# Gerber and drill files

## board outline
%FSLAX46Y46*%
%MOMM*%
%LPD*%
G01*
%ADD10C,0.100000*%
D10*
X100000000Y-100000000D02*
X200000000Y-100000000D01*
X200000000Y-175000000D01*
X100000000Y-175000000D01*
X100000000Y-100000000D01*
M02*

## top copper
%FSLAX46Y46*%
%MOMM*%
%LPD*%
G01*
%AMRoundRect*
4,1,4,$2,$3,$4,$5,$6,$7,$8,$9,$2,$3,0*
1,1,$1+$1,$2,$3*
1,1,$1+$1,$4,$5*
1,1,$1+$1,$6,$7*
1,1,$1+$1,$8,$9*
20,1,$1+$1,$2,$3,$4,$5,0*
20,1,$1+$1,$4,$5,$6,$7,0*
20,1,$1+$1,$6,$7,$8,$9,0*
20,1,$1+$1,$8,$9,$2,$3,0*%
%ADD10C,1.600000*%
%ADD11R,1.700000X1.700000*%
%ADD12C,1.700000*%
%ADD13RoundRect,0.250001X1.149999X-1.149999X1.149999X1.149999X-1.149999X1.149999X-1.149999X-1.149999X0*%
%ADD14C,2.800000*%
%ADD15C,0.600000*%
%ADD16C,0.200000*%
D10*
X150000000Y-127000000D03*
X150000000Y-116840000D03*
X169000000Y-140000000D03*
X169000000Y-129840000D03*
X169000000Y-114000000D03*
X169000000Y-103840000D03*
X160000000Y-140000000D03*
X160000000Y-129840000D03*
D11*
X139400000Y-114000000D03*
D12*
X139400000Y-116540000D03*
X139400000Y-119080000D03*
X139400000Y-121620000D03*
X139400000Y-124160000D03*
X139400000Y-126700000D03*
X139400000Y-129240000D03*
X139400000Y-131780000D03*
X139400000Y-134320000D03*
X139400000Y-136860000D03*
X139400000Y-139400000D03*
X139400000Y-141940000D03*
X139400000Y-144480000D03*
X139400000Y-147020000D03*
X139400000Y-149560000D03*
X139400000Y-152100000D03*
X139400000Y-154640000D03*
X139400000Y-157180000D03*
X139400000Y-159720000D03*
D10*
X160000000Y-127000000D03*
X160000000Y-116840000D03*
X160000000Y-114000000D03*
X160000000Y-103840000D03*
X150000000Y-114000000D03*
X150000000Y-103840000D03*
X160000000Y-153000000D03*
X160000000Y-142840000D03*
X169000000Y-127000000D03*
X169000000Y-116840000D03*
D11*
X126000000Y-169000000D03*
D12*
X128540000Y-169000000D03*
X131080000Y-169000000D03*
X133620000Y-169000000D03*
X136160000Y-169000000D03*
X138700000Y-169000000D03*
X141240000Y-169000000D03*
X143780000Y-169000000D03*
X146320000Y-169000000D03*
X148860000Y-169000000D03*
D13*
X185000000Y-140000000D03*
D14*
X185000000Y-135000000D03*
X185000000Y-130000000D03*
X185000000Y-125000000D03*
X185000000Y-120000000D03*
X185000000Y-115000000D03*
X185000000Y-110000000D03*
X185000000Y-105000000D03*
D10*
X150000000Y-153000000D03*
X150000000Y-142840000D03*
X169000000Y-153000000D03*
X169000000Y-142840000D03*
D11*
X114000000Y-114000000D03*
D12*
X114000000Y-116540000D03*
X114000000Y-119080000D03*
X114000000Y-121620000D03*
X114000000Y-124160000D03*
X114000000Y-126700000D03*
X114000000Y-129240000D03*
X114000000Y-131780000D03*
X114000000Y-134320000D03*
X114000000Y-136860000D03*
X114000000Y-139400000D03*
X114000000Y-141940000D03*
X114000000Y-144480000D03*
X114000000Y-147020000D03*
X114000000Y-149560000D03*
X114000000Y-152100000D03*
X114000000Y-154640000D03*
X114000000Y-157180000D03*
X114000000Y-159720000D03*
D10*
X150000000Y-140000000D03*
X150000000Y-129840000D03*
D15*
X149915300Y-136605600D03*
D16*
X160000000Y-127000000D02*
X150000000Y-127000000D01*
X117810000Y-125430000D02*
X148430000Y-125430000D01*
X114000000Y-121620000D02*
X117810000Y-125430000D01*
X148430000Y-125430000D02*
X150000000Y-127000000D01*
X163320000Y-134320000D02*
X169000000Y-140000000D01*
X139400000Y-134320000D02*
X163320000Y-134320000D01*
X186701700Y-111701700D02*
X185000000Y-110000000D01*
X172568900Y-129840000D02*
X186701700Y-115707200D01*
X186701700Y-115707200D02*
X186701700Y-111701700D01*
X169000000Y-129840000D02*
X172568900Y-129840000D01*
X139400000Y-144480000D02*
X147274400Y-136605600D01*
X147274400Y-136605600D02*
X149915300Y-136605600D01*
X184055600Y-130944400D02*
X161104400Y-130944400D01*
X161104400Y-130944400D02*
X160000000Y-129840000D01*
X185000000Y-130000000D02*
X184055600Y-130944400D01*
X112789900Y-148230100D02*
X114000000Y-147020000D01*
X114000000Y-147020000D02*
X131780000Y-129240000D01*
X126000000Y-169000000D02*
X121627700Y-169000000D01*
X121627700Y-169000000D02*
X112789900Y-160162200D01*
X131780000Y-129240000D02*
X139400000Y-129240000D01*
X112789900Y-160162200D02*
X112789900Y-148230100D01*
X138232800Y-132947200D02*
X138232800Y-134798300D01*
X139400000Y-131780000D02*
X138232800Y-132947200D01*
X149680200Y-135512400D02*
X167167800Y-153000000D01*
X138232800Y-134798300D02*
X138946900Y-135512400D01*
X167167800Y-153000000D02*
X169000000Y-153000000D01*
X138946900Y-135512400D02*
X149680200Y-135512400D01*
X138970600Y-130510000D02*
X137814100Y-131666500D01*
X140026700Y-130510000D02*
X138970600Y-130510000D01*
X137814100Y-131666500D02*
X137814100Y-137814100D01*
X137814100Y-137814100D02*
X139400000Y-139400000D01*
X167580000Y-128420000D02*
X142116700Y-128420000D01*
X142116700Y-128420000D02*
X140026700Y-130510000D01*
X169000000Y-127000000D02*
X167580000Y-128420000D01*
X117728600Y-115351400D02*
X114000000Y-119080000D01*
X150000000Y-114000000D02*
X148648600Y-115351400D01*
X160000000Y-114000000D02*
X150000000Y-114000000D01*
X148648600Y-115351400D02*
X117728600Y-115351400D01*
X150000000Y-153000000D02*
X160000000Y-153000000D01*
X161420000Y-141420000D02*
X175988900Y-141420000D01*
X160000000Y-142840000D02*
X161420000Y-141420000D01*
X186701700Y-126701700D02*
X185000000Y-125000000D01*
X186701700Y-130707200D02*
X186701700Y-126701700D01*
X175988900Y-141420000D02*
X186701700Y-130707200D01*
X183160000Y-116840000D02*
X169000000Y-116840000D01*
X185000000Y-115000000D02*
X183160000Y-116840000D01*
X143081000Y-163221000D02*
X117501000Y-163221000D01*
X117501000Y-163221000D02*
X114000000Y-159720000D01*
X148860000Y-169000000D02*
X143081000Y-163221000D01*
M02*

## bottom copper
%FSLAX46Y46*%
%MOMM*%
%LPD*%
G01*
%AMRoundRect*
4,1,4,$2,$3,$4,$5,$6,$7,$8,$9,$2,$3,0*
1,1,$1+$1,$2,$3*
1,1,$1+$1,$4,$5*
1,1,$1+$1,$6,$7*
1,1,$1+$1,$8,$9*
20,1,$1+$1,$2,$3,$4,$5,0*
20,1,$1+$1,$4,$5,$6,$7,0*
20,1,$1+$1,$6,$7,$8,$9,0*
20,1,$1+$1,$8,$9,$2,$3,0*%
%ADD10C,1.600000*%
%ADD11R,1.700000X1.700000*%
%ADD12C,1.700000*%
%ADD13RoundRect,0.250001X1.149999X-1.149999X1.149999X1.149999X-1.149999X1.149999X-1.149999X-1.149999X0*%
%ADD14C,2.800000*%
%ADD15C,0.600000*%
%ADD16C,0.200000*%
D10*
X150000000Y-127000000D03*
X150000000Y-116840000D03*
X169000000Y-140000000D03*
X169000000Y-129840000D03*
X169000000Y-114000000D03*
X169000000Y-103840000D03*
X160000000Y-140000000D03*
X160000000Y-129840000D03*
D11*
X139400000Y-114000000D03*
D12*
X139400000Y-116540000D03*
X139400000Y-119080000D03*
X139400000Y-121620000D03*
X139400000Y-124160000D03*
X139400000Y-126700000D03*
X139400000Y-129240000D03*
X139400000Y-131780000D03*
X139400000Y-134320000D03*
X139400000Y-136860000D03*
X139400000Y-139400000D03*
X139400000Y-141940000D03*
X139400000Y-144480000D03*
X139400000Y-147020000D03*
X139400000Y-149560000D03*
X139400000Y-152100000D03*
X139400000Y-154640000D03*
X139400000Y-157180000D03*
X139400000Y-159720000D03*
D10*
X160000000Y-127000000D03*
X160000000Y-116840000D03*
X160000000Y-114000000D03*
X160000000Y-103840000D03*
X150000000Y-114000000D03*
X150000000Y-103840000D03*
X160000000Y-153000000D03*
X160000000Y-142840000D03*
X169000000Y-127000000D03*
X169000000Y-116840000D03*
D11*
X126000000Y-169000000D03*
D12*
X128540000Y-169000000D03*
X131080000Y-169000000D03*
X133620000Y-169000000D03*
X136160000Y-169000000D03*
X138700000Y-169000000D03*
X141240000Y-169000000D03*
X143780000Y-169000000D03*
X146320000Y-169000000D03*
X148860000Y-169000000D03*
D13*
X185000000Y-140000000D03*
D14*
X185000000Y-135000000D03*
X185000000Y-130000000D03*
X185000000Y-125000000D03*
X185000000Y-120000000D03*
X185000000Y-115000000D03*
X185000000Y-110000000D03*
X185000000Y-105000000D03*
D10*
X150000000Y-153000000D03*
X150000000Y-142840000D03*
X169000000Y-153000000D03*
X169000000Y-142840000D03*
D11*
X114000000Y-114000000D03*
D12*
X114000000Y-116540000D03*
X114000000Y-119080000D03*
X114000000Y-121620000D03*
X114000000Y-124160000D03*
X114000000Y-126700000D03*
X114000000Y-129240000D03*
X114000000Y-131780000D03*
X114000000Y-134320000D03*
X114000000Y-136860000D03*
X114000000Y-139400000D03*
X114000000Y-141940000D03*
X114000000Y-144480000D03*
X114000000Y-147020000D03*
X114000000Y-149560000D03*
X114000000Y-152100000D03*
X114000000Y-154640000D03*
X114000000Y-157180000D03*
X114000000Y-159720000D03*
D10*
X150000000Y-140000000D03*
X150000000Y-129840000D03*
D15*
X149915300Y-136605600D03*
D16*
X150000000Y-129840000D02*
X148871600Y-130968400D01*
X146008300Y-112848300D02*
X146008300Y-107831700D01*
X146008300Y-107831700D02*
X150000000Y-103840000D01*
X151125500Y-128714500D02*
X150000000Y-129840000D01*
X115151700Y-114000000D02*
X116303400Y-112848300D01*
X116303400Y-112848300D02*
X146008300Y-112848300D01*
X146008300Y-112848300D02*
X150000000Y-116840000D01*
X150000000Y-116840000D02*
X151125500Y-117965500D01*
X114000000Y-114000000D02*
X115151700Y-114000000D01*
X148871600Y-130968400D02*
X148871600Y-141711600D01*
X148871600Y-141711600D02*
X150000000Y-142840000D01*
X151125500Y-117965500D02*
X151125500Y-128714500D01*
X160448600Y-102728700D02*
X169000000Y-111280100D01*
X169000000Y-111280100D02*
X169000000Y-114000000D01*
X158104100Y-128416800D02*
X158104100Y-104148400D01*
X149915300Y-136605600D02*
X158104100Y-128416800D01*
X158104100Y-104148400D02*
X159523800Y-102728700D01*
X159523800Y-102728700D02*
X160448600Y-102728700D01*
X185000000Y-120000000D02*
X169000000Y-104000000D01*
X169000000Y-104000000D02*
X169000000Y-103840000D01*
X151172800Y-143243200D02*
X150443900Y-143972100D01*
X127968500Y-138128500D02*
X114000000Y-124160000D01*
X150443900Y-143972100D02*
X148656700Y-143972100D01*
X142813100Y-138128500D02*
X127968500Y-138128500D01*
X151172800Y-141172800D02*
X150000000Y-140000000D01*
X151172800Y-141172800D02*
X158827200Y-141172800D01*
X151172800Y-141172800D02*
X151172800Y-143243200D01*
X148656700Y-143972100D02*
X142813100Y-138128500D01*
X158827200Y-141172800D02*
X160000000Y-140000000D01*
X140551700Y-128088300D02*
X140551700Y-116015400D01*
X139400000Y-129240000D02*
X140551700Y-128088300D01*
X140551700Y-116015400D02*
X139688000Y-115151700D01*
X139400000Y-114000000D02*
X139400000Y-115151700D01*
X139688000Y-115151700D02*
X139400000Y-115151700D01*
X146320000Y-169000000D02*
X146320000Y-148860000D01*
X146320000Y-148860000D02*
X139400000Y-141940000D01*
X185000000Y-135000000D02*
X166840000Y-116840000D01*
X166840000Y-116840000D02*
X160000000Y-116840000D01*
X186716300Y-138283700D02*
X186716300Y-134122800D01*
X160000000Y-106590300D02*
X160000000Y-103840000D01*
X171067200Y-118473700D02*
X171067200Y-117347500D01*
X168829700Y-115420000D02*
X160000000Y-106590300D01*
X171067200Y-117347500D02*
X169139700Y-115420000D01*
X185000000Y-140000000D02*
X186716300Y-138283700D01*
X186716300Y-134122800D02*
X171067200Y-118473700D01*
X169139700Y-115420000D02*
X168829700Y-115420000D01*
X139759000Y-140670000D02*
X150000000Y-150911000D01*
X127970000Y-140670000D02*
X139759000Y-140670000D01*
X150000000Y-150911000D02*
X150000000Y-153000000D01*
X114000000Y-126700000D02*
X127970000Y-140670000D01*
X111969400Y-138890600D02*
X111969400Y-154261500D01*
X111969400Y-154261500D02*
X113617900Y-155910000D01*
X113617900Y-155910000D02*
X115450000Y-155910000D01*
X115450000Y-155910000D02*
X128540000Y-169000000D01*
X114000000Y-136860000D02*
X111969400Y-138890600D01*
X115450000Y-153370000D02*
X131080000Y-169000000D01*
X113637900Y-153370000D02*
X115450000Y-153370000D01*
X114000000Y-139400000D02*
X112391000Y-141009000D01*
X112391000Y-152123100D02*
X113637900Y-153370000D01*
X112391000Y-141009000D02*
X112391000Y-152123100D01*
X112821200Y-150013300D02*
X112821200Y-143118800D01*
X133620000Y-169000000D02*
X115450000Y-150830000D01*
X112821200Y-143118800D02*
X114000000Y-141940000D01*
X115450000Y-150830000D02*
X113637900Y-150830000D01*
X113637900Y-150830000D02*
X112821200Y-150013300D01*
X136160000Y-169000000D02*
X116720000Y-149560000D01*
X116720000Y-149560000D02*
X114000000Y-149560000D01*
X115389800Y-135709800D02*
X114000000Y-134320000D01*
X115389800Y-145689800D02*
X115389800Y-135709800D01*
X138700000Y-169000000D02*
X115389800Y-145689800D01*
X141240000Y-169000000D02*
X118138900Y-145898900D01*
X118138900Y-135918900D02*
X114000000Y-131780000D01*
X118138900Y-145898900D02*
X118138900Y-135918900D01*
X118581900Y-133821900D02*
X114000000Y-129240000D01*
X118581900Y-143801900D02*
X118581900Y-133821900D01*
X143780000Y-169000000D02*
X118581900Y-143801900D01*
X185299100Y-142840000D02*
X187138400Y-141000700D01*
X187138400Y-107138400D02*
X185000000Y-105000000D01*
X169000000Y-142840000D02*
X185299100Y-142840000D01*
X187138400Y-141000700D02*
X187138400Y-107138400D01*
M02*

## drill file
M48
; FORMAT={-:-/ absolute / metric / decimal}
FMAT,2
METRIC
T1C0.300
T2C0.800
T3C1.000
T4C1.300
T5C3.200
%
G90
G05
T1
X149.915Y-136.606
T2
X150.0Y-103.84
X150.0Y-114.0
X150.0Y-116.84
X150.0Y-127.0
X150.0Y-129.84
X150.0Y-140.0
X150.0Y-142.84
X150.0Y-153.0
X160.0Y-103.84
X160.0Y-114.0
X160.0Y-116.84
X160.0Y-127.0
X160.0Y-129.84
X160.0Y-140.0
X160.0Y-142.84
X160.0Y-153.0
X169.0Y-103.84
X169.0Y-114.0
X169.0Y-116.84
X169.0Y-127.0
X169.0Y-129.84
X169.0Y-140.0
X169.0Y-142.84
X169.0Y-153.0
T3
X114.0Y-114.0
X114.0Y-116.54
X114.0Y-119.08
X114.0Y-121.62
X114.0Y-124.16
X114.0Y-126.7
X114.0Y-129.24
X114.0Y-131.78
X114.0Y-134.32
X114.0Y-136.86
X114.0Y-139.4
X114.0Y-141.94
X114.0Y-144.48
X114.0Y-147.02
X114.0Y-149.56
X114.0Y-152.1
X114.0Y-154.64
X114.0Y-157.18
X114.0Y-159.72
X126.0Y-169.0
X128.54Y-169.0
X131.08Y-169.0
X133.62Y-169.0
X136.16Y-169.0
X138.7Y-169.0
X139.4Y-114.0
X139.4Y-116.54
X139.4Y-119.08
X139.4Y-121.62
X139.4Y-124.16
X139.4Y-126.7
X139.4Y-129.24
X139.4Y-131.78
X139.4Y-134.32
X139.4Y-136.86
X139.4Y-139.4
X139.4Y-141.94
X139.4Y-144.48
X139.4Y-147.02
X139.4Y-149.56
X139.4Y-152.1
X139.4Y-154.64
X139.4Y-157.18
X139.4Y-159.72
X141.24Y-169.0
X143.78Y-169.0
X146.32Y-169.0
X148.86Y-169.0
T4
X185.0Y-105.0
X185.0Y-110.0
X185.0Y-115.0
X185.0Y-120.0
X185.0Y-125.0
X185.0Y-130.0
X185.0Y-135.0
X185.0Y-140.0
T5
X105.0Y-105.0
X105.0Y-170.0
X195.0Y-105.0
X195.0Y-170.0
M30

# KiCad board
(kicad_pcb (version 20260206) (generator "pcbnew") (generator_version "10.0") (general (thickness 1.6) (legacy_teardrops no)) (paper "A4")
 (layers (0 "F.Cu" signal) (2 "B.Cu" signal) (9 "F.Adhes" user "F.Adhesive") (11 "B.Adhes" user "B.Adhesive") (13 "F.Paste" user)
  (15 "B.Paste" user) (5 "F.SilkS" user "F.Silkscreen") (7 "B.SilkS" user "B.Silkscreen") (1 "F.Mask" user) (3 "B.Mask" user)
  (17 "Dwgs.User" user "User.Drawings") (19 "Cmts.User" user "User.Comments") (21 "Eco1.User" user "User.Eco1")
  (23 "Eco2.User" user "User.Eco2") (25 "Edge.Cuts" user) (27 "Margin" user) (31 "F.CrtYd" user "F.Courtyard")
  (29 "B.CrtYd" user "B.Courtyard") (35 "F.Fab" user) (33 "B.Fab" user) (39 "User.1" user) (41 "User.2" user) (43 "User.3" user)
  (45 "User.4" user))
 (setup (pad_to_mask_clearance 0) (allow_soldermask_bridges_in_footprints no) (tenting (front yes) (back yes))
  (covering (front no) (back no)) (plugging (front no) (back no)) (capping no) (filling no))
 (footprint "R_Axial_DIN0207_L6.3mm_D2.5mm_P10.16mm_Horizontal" (layer "F.Cu") (at 150 127 90)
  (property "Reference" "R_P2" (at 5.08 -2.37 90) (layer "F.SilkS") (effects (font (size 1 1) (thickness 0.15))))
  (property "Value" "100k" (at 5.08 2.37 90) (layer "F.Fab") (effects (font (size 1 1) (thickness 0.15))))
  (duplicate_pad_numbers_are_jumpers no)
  (pad "1" thru_hole circle (at 0 0 90) (size 1.6 1.6) (drill 0.8) (layers "*.Cu" "*.Mask") (remove_unused_layers no) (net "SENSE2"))
  (pad "2" thru_hole circle (at 10.16 0 90) (size 1.6 1.6) (drill 0.8) (layers "*.Cu" "*.Mask") (remove_unused_layers no) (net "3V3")))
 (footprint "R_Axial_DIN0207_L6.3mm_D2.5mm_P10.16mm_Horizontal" (layer "F.Cu") (at 169 140 90)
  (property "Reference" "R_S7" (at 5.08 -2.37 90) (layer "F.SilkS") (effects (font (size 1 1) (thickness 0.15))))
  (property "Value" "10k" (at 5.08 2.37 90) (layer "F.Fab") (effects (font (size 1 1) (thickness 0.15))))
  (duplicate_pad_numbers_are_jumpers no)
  (pad "1" thru_hole circle (at 0 0 90) (size 1.6 1.6) (drill 0.8) (layers "*.Cu" "*.Mask") (remove_unused_layers no) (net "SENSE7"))
  (pad "2" thru_hole circle (at 10.16 0 90) (size 1.6 1.6) (drill 0.8) (layers "*.Cu" "*.Mask") (remove_unused_layers no) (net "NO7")))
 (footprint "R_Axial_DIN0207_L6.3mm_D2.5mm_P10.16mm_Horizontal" (layer "F.Cu") (at 169 114 90)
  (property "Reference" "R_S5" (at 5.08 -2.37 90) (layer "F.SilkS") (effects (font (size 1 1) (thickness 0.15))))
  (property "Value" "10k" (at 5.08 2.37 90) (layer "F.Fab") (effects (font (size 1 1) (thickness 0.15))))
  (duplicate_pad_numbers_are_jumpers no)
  (pad "1" thru_hole circle (at 0 0 90) (size 1.6 1.6) (drill 0.8) (layers "*.Cu" "*.Mask") (remove_unused_layers no) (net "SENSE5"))
  (pad "2" thru_hole circle (at 10.16 0 90) (size 1.6 1.6) (drill 0.8) (layers "*.Cu" "*.Mask") (remove_unused_layers no) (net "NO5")))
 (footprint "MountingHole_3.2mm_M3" (layer "F.Cu") (at 105 170)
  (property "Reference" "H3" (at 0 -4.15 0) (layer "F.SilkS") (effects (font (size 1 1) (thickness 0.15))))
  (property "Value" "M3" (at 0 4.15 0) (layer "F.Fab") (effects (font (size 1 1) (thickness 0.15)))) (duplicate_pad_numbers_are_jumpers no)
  (pad "" np_thru_hole circle (at 0 0) (size 3.2 3.2) (drill 3.2) (layers "*.Cu" "*.Mask")))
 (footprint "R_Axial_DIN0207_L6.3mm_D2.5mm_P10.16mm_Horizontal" (layer "F.Cu") (at 160 140 90)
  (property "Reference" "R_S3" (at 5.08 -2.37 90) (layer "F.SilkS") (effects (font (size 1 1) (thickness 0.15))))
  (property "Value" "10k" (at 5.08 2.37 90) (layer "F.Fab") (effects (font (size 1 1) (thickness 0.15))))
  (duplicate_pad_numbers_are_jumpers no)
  (pad "1" thru_hole circle (at 0 0 90) (size 1.6 1.6) (drill 0.8) (layers "*.Cu" "*.Mask") (remove_unused_layers no) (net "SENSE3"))
  (pad "2" thru_hole circle (at 10.16 0 90) (size 1.6 1.6) (drill 0.8) (layers "*.Cu" "*.Mask") (remove_unused_layers no) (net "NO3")))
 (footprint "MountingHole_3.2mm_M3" (layer "F.Cu") (at 195 170)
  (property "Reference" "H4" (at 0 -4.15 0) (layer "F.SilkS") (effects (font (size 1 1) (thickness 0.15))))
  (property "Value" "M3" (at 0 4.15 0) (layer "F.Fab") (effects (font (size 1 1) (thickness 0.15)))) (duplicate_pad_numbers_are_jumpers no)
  (pad "" np_thru_hole circle (at 0 0) (size 3.2 3.2) (drill 3.2) (layers "*.Cu" "*.Mask")))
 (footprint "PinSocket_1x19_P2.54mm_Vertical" (layer "F.Cu") (at 139.4 114)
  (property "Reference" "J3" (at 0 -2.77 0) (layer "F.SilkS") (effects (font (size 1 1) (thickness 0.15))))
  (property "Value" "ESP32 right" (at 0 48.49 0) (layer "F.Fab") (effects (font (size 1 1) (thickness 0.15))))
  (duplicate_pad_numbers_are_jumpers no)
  (pad "1" thru_hole rect (at 0 0) (size 1.7 1.7) (drill 1) (layers "*.Cu" "*.Mask") (remove_unused_layers no) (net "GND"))
  (pad "2" thru_hole circle (at 0 2.54) (size 1.7 1.7) (drill 1) (layers "*.Cu" "*.Mask") (remove_unused_layers no))
  (pad "3" thru_hole circle (at 0 5.08) (size 1.7 1.7) (drill 1) (layers "*.Cu" "*.Mask") (remove_unused_layers no))
  (pad "4" thru_hole circle (at 0 7.62) (size 1.7 1.7) (drill 1) (layers "*.Cu" "*.Mask") (remove_unused_layers no))
  (pad "5" thru_hole circle (at 0 10.16) (size 1.7 1.7) (drill 1) (layers "*.Cu" "*.Mask") (remove_unused_layers no))
  (pad "6" thru_hole circle (at 0 12.7) (size 1.7 1.7) (drill 1) (layers "*.Cu" "*.Mask") (remove_unused_layers no))
  (pad "7" thru_hole circle (at 0 15.24) (size 1.7 1.7) (drill 1) (layers "*.Cu" "*.Mask") (remove_unused_layers no) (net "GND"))
  (pad "8" thru_hole circle (at 0 17.78) (size 1.7 1.7) (drill 1) (layers "*.Cu" "*.Mask") (remove_unused_layers no) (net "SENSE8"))
  (pad "9" thru_hole circle (at 0 20.32) (size 1.7 1.7) (drill 1) (layers "*.Cu" "*.Mask") (remove_unused_layers no) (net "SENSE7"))
  (pad "10" thru_hole circle (at 0 22.86) (size 1.7 1.7) (drill 1) (layers "*.Cu" "*.Mask") (remove_unused_layers no))
  (pad "11" thru_hole circle (at 0 25.4) (size 1.7 1.7) (drill 1) (layers "*.Cu" "*.Mask") (remove_unused_layers no) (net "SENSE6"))
  (pad "12" thru_hole circle (at 0 27.94) (size 1.7 1.7) (drill 1) (layers "*.Cu" "*.Mask") (remove_unused_layers no) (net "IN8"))
  (pad "13" thru_hole circle (at 0 30.48) (size 1.7 1.7) (drill 1) (layers "*.Cu" "*.Mask") (remove_unused_layers no) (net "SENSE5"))
  (pad "14" thru_hole circle (at 0 33.02) (size 1.7 1.7) (drill 1) (layers "*.Cu" "*.Mask") (remove_unused_layers no))
  (pad "15" thru_hole circle (at 0 35.56) (size 1.7 1.7) (drill 1) (layers "*.Cu" "*.Mask") (remove_unused_layers no))
  (pad "16" thru_hole circle (at 0 38.1) (size 1.7 1.7) (drill 1) (layers "*.Cu" "*.Mask") (remove_unused_layers no))
  (pad "17" thru_hole circle (at 0 40.64) (size 1.7 1.7) (drill 1) (layers "*.Cu" "*.Mask") (remove_unused_layers no))
  (pad "18" thru_hole circle (at 0 43.18) (size 1.7 1.7) (drill 1) (layers "*.Cu" "*.Mask") (remove_unused_layers no))
  (pad "19" thru_hole circle (at 0 45.72) (size 1.7 1.7) (drill 1) (layers "*.Cu" "*.Mask") (remove_unused_layers no)))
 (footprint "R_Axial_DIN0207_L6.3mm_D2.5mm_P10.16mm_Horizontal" (layer "F.Cu") (at 160 127 90)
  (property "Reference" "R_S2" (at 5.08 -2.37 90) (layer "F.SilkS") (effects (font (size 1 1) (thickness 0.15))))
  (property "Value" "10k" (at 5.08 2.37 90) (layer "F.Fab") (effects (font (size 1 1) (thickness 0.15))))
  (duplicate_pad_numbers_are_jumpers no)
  (pad "1" thru_hole circle (at 0 0 90) (size 1.6 1.6) (drill 0.8) (layers "*.Cu" "*.Mask") (remove_unused_layers no) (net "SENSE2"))
  (pad "2" thru_hole circle (at 10.16 0 90) (size 1.6 1.6) (drill 0.8) (layers "*.Cu" "*.Mask") (remove_unused_layers no) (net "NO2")))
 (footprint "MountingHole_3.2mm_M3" (layer "F.Cu") (at 195 105)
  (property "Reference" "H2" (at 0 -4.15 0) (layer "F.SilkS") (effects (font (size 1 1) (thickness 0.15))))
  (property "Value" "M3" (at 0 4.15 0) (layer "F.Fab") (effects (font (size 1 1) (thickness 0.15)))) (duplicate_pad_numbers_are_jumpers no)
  (pad "" np_thru_hole circle (at 0 0) (size 3.2 3.2) (drill 3.2) (layers "*.Cu" "*.Mask")))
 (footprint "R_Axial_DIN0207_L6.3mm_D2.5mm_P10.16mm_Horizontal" (layer "F.Cu") (at 160 114 90)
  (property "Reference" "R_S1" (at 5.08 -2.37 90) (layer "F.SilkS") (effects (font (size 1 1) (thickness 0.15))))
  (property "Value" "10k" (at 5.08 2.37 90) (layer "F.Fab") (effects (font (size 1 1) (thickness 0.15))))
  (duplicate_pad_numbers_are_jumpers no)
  (pad "1" thru_hole circle (at 0 0 90) (size 1.6 1.6) (drill 0.8) (layers "*.Cu" "*.Mask") (remove_unused_layers no) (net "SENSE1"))
  (pad "2" thru_hole circle (at 10.16 0 90) (size 1.6 1.6) (drill 0.8) (layers "*.Cu" "*.Mask") (remove_unused_layers no) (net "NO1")))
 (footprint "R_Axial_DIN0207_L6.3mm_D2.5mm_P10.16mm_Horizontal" (layer "F.Cu") (at 150 114 90)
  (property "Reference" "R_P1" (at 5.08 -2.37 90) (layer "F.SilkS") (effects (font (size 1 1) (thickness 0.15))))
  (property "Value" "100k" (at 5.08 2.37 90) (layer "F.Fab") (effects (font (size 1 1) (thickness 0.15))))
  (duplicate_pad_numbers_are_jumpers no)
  (pad "1" thru_hole circle (at 0 0 90) (size 1.6 1.6) (drill 0.8) (layers "*.Cu" "*.Mask") (remove_unused_layers no) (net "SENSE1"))
  (pad "2" thru_hole circle (at 10.16 0 90) (size 1.6 1.6) (drill 0.8) (layers "*.Cu" "*.Mask") (remove_unused_layers no) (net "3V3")))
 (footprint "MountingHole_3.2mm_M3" (layer "F.Cu") (at 105 105)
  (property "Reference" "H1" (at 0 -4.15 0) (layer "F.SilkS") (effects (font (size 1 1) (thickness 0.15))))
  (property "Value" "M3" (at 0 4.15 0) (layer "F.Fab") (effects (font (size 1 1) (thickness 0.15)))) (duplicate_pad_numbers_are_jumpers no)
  (pad "" np_thru_hole circle (at 0 0) (size 3.2 3.2) (drill 3.2) (layers "*.Cu" "*.Mask")))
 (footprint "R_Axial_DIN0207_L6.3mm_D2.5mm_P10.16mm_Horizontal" (layer "F.Cu") (at 160 153 90)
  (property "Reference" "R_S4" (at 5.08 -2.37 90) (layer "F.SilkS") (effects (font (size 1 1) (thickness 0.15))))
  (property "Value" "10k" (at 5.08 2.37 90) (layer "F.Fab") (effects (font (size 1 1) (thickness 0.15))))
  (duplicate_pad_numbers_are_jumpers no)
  (pad "1" thru_hole circle (at 0 0 90) (size 1.6 1.6) (drill 0.8) (layers "*.Cu" "*.Mask") (remove_unused_layers no) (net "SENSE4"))
  (pad "2" thru_hole circle (at 10.16 0 90) (size 1.6 1.6) (drill 0.8) (layers "*.Cu" "*.Mask") (remove_unused_layers no) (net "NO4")))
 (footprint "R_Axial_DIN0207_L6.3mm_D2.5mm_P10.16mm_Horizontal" (layer "F.Cu") (at 169 127 90)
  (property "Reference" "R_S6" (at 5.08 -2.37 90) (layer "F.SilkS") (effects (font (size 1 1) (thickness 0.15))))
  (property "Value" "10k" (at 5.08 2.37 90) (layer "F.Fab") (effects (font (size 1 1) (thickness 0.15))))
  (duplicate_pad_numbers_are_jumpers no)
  (pad "1" thru_hole circle (at 0 0 90) (size 1.6 1.6) (drill 0.8) (layers "*.Cu" "*.Mask") (remove_unused_layers no) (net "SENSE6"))
  (pad "2" thru_hole circle (at 10.16 0 90) (size 1.6 1.6) (drill 0.8) (layers "*.Cu" "*.Mask") (remove_unused_layers no) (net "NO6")))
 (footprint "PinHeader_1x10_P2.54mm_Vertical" (layer "F.Cu") (at 126 169 90)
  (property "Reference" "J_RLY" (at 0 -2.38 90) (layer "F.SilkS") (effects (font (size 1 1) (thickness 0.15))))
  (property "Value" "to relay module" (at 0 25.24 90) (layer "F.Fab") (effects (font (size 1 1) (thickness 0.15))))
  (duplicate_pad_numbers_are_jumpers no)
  (pad "1" thru_hole rect (at 0 0 90) (size 1.7 1.7) (drill 1) (layers "*.Cu" "*.Mask") (remove_unused_layers no) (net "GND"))
  (pad "2" thru_hole circle (at 0 2.54 90) (size 1.7 1.7) (drill 1) (layers "*.Cu" "*.Mask") (remove_unused_layers no) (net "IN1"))
  (pad "3" thru_hole circle (at 0 5.08 90) (size 1.7 1.7) (drill 1) (layers "*.Cu" "*.Mask") (remove_unused_layers no) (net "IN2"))
  (pad "4" thru_hole circle (at 0 7.62 90) (size 1.7 1.7) (drill 1) (layers "*.Cu" "*.Mask") (remove_unused_layers no) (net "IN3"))
  (pad "5" thru_hole circle (at 0 10.16 90) (size 1.7 1.7) (drill 1) (layers "*.Cu" "*.Mask") (remove_unused_layers no) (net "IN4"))
  (pad "6" thru_hole circle (at 0 12.7 90) (size 1.7 1.7) (drill 1) (layers "*.Cu" "*.Mask") (remove_unused_layers no) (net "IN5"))
  (pad "7" thru_hole circle (at 0 15.24 90) (size 1.7 1.7) (drill 1) (layers "*.Cu" "*.Mask") (remove_unused_layers no) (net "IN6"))
  (pad "8" thru_hole circle (at 0 17.78 90) (size 1.7 1.7) (drill 1) (layers "*.Cu" "*.Mask") (remove_unused_layers no) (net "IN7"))
  (pad "9" thru_hole circle (at 0 20.32 90) (size 1.7 1.7) (drill 1) (layers "*.Cu" "*.Mask") (remove_unused_layers no) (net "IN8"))
  (pad "10" thru_hole circle (at 0 22.86 90) (size 1.7 1.7) (drill 1) (layers "*.Cu" "*.Mask") (remove_unused_layers no) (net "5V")))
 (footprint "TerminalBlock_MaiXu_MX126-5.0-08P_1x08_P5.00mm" (layer "F.Cu") (at 185 140 90)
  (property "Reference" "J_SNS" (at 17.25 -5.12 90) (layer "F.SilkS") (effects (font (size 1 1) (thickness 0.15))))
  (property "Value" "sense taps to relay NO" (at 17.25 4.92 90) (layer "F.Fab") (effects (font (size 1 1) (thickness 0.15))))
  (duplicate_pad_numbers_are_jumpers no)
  (pad "1" thru_hole roundrect (at 0 0 90) (size 2.8 2.8) (drill 1.3) (layers "*.Cu" "*.Mask") (remove_unused_layers no)
   (roundrect_rratio 0.089286) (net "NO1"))
  (pad "2" thru_hole circle (at 5 0 90) (size 2.8 2.8) (drill 1.3) (layers "*.Cu" "*.Mask") (remove_unused_layers no) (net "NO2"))
  (pad "3" thru_hole circle (at 10 0 90) (size 2.8 2.8) (drill 1.3) (layers "*.Cu" "*.Mask") (remove_unused_layers no) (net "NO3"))
  (pad "4" thru_hole circle (at 15 0 90) (size 2.8 2.8) (drill 1.3) (layers "*.Cu" "*.Mask") (remove_unused_layers no) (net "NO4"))
  (pad "5" thru_hole circle (at 20 0 90) (size 2.8 2.8) (drill 1.3) (layers "*.Cu" "*.Mask") (remove_unused_layers no) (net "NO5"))
  (pad "6" thru_hole circle (at 25 0 90) (size 2.8 2.8) (drill 1.3) (layers "*.Cu" "*.Mask") (remove_unused_layers no) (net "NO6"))
  (pad "7" thru_hole circle (at 30 0 90) (size 2.8 2.8) (drill 1.3) (layers "*.Cu" "*.Mask") (remove_unused_layers no) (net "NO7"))
  (pad "8" thru_hole circle (at 35 0 90) (size 2.8 2.8) (drill 1.3) (layers "*.Cu" "*.Mask") (remove_unused_layers no) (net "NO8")))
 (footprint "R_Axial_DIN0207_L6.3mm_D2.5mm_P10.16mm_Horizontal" (layer "F.Cu") (at 150 153 90)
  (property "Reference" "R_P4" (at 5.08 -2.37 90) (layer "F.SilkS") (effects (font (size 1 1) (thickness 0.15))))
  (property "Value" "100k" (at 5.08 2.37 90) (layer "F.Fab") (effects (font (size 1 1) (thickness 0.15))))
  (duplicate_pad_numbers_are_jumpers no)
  (pad "1" thru_hole circle (at 0 0 90) (size 1.6 1.6) (drill 0.8) (layers "*.Cu" "*.Mask") (remove_unused_layers no) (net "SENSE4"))
  (pad "2" thru_hole circle (at 10.16 0 90) (size 1.6 1.6) (drill 0.8) (layers "*.Cu" "*.Mask") (remove_unused_layers no) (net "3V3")))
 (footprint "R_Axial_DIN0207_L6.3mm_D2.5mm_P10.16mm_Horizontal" (layer "F.Cu") (at 169 153 90)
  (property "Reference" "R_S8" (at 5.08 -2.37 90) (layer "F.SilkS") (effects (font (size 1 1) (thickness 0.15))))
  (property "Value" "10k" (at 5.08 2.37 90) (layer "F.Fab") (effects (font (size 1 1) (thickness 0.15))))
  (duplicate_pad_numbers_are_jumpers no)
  (pad "1" thru_hole circle (at 0 0 90) (size 1.6 1.6) (drill 0.8) (layers "*.Cu" "*.Mask") (remove_unused_layers no) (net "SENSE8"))
  (pad "2" thru_hole circle (at 10.16 0 90) (size 1.6 1.6) (drill 0.8) (layers "*.Cu" "*.Mask") (remove_unused_layers no) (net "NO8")))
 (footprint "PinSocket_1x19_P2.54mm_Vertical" (layer "F.Cu") (at 114 114)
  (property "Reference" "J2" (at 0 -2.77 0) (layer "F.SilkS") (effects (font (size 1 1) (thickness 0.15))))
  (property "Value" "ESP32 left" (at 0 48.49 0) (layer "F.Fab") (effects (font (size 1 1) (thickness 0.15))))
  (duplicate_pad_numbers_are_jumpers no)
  (pad "1" thru_hole rect (at 0 0) (size 1.7 1.7) (drill 1) (layers "*.Cu" "*.Mask") (remove_unused_layers no) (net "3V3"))
  (pad "2" thru_hole circle (at 0 2.54) (size 1.7 1.7) (drill 1) (layers "*.Cu" "*.Mask") (remove_unused_layers no))
  (pad "3" thru_hole circle (at 0 5.08) (size 1.7 1.7) (drill 1) (layers "*.Cu" "*.Mask") (remove_unused_layers no) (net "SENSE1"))
  (pad "4" thru_hole circle (at 0 7.62) (size 1.7 1.7) (drill 1) (layers "*.Cu" "*.Mask") (remove_unused_layers no) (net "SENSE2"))
  (pad "5" thru_hole circle (at 0 10.16) (size 1.7 1.7) (drill 1) (layers "*.Cu" "*.Mask") (remove_unused_layers no) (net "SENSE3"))
  (pad "6" thru_hole circle (at 0 12.7) (size 1.7 1.7) (drill 1) (layers "*.Cu" "*.Mask") (remove_unused_layers no) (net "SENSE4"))
  (pad "7" thru_hole circle (at 0 15.24) (size 1.7 1.7) (drill 1) (layers "*.Cu" "*.Mask") (remove_unused_layers no) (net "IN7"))
  (pad "8" thru_hole circle (at 0 17.78) (size 1.7 1.7) (drill 1) (layers "*.Cu" "*.Mask") (remove_unused_layers no) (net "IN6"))
  (pad "9" thru_hole circle (at 0 20.32) (size 1.7 1.7) (drill 1) (layers "*.Cu" "*.Mask") (remove_unused_layers no) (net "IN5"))
  (pad "10" thru_hole circle (at 0 22.86) (size 1.7 1.7) (drill 1) (layers "*.Cu" "*.Mask") (remove_unused_layers no) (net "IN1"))
  (pad "11" thru_hole circle (at 0 25.4) (size 1.7 1.7) (drill 1) (layers "*.Cu" "*.Mask") (remove_unused_layers no) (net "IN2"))
  (pad "12" thru_hole circle (at 0 27.94) (size 1.7 1.7) (drill 1) (layers "*.Cu" "*.Mask") (remove_unused_layers no) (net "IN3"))
  (pad "13" thru_hole circle (at 0 30.48) (size 1.7 1.7) (drill 1) (layers "*.Cu" "*.Mask") (remove_unused_layers no))
  (pad "14" thru_hole circle (at 0 33.02) (size 1.7 1.7) (drill 1) (layers "*.Cu" "*.Mask") (remove_unused_layers no) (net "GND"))
  (pad "15" thru_hole circle (at 0 35.56) (size 1.7 1.7) (drill 1) (layers "*.Cu" "*.Mask") (remove_unused_layers no) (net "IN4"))
  (pad "16" thru_hole circle (at 0 38.1) (size 1.7 1.7) (drill 1) (layers "*.Cu" "*.Mask") (remove_unused_layers no))
  (pad "17" thru_hole circle (at 0 40.64) (size 1.7 1.7) (drill 1) (layers "*.Cu" "*.Mask") (remove_unused_layers no))
  (pad "18" thru_hole circle (at 0 43.18) (size 1.7 1.7) (drill 1) (layers "*.Cu" "*.Mask") (remove_unused_layers no))
  (pad "19" thru_hole circle (at 0 45.72) (size 1.7 1.7) (drill 1) (layers "*.Cu" "*.Mask") (remove_unused_layers no) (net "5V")))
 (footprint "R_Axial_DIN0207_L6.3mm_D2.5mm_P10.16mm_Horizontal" (layer "F.Cu") (at 150 140 90)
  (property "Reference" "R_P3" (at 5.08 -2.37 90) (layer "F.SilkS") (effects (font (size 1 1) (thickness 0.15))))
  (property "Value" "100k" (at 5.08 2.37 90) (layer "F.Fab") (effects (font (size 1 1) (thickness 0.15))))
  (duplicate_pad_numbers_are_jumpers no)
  (pad "1" thru_hole circle (at 0 0 90) (size 1.6 1.6) (drill 0.8) (layers "*.Cu" "*.Mask") (remove_unused_layers no) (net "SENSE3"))
  (pad "2" thru_hole circle (at 10.16 0 90) (size 1.6 1.6) (drill 0.8) (layers "*.Cu" "*.Mask") (remove_unused_layers no) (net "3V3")))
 (gr_rect (start 100 100) (end 200 175) (stroke (width 0.1) (type default)) (fill no) (layer "Edge.Cuts"))
 (segment (start 160 127) (end 150 127) (width 0.2) (layer "F.Cu") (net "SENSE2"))
 (segment (start 117.81 125.43) (end 148.43 125.43) (width 0.2) (layer "F.Cu") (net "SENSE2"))
 (segment (start 114 121.62) (end 117.81 125.43) (width 0.2) (layer "F.Cu") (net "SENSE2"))
 (segment (start 148.43 125.43) (end 150 127) (width 0.2) (layer "F.Cu") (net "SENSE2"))
 (segment (start 150 129.84) (end 148.8716 130.9684) (width 0.2) (layer "B.Cu") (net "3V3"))
 (segment (start 146.0083 112.8483) (end 146.0083 107.8317) (width 0.2) (layer "B.Cu") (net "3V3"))
 (segment (start 146.0083 107.8317) (end 150 103.84) (width 0.2) (layer "B.Cu") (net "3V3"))
 (segment (start 151.1255 128.7145) (end 150 129.84) (width 0.2) (layer "B.Cu") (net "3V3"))
 (segment (start 115.1517 114) (end 116.3034 112.8483) (width 0.2) (layer "B.Cu") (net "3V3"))
 (segment (start 116.3034 112.8483) (end 146.0083 112.8483) (width 0.2) (layer "B.Cu") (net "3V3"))
 (segment (start 146.0083 112.8483) (end 150 116.84) (width 0.2) (layer "B.Cu") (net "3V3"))
 (segment (start 150 116.84) (end 151.1255 117.9655) (width 0.2) (layer "B.Cu") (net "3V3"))
 (segment (start 114 114) (end 115.1517 114) (width 0.2) (layer "B.Cu") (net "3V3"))
 (segment (start 148.8716 130.9684) (end 148.8716 141.7116) (width 0.2) (layer "B.Cu") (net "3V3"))
 (segment (start 148.8716 141.7116) (end 150 142.84) (width 0.2) (layer "B.Cu") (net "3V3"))
 (segment (start 151.1255 117.9655) (end 151.1255 128.7145) (width 0.2) (layer "B.Cu") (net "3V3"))
 (segment (start 163.32 134.32) (end 169 140) (width 0.2) (layer "F.Cu") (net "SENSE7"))
 (segment (start 139.4 134.32) (end 163.32 134.32) (width 0.2) (layer "F.Cu") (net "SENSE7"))
 (segment (start 186.7017 111.7017) (end 185 110) (width 0.2) (layer "F.Cu") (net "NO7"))
 (segment (start 172.5689 129.84) (end 186.7017 115.7072) (width 0.2) (layer "F.Cu") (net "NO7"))
 (segment (start 186.7017 115.7072) (end 186.7017 111.7017) (width 0.2) (layer "F.Cu") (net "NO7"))
 (segment (start 169 129.84) (end 172.5689 129.84) (width 0.2) (layer "F.Cu") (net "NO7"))
 (segment (start 139.4 144.48) (end 147.2744 136.6056) (width 0.2) (layer "F.Cu") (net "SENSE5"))
 (segment (start 147.2744 136.6056) (end 149.9153 136.6056) (width 0.2) (layer "F.Cu") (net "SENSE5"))
 (via (at 149.9153 136.6056) (size 0.6) (drill 0.3) (layers "F.Cu" "B.Cu") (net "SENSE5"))
 (segment (start 160.4486 102.7287) (end 169 111.2801) (width 0.2) (layer "B.Cu") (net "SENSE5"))
 (segment (start 169 111.2801) (end 169 114) (width 0.2) (layer "B.Cu") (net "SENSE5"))
 (segment (start 158.1041 128.4168) (end 158.1041 104.1484) (width 0.2) (layer "B.Cu") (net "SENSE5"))
 (segment (start 149.9153 136.6056) (end 158.1041 128.4168) (width 0.2) (layer "B.Cu") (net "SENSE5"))
 (segment (start 158.1041 104.1484) (end 159.5238 102.7287) (width 0.2) (layer "B.Cu") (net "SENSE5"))
 (segment (start 159.5238 102.7287) (end 160.4486 102.7287) (width 0.2) (layer "B.Cu") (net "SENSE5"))
 (segment (start 185 120) (end 169 104) (width 0.2) (layer "B.Cu") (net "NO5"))
 (segment (start 169 104) (end 169 103.84) (width 0.2) (layer "B.Cu") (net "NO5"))
 (segment (start 151.1728 143.2432) (end 150.4439 143.9721) (width 0.2) (layer "B.Cu") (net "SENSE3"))
 (segment (start 127.9685 138.1285) (end 114 124.16) (width 0.2) (layer "B.Cu") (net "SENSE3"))
 (segment (start 150.4439 143.9721) (end 148.6567 143.9721) (width 0.2) (layer "B.Cu") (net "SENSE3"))
 (segment (start 142.8131 138.1285) (end 127.9685 138.1285) (width 0.2) (layer "B.Cu") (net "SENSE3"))
 (segment (start 151.1728 141.1728) (end 150 140) (width 0.2) (layer "B.Cu") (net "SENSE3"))
 (segment (start 151.1728 141.1728) (end 158.8272 141.1728) (width 0.2) (layer "B.Cu") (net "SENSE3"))
 (segment (start 151.1728 141.1728) (end 151.1728 143.2432) (width 0.2) (layer "B.Cu") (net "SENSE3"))
 (segment (start 148.6567 143.9721) (end 142.8131 138.1285) (width 0.2) (layer "B.Cu") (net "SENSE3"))
 (segment (start 158.8272 141.1728) (end 160 140) (width 0.2) (layer "B.Cu") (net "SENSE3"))
 (segment (start 184.0556 130.9444) (end 161.1044 130.9444) (width 0.2) (layer "F.Cu") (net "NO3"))
 (segment (start 161.1044 130.9444) (end 160 129.84) (width 0.2) (layer "F.Cu") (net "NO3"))
 (segment (start 185 130) (end 184.0556 130.9444) (width 0.2) (layer "F.Cu") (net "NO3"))
 (segment (start 112.7899 148.2301) (end 114 147.02) (width 0.2) (layer "F.Cu") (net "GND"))
 (segment (start 114 147.02) (end 131.78 129.24) (width 0.2) (layer "F.Cu") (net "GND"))
 (segment (start 126 169) (end 121.6277 169) (width 0.2) (layer "F.Cu") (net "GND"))
 (segment (start 121.6277 169) (end 112.7899 160.1622) (width 0.2) (layer "F.Cu") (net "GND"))
 (segment (start 131.78 129.24) (end 139.4 129.24) (width 0.2) (layer "F.Cu") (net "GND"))
 (segment (start 112.7899 160.1622) (end 112.7899 148.2301) (width 0.2) (layer "F.Cu") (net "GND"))
 (segment (start 140.5517 128.0883) (end 140.5517 116.0154) (width 0.2) (layer "B.Cu") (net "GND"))
 (segment (start 139.4 129.24) (end 140.5517 128.0883) (width 0.2) (layer "B.Cu") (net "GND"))
 (segment (start 140.5517 116.0154) (end 139.688 115.1517) (width 0.2) (layer "B.Cu") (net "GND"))
 (segment (start 139.4 114) (end 139.4 115.1517) (width 0.2) (layer "B.Cu") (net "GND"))
 (segment (start 139.688 115.1517) (end 139.4 115.1517) (width 0.2) (layer "B.Cu") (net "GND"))
 (segment (start 138.2328 132.9472) (end 138.2328 134.7983) (width 0.2) (layer "F.Cu") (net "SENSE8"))
 (segment (start 139.4 131.78) (end 138.2328 132.9472) (width 0.2) (layer "F.Cu") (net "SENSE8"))
 (segment (start 149.6802 135.5124) (end 167.1678 153) (width 0.2) (layer "F.Cu") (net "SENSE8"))
 (segment (start 138.2328 134.7983) (end 138.9469 135.5124) (width 0.2) (layer "F.Cu") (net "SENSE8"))
 (segment (start 167.1678 153) (end 169 153) (width 0.2) (layer "F.Cu") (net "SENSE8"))
 (segment (start 138.9469 135.5124) (end 149.6802 135.5124) (width 0.2) (layer "F.Cu") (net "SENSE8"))
 (segment (start 138.9706 130.51) (end 137.8141 131.6665) (width 0.2) (layer "F.Cu") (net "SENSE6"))
 (segment (start 140.0267 130.51) (end 138.9706 130.51) (width 0.2) (layer "F.Cu") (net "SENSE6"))
 (segment (start 137.8141 131.6665) (end 137.8141 137.8141) (width 0.2) (layer "F.Cu") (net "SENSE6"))
 (segment (start 137.8141 137.8141) (end 139.4 139.4) (width 0.2) (layer "F.Cu") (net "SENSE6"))
 (segment (start 167.58 128.42) (end 142.1167 128.42) (width 0.2) (layer "F.Cu") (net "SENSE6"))
 (segment (start 142.1167 128.42) (end 140.0267 130.51) (width 0.2) (layer "F.Cu") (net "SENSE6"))
 (segment (start 169 127) (end 167.58 128.42) (width 0.2) (layer "F.Cu") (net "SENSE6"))
 (segment (start 146.32 169) (end 146.32 148.86) (width 0.2) (layer "B.Cu") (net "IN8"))
 (segment (start 146.32 148.86) (end 139.4 141.94) (width 0.2) (layer "B.Cu") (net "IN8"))
 (segment (start 185 135) (end 166.84 116.84) (width 0.2) (layer "B.Cu") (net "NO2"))
 (segment (start 166.84 116.84) (end 160 116.84) (width 0.2) (layer "B.Cu") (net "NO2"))
 (segment (start 117.7286 115.3514) (end 114 119.08) (width 0.2) (layer "F.Cu") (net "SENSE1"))
 (segment (start 150 114) (end 148.6486 115.3514) (width 0.2) (layer "F.Cu") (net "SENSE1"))
 (segment (start 160 114) (end 150 114) (width 0.2) (layer "F.Cu") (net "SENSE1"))
 (segment (start 148.6486 115.3514) (end 117.7286 115.3514) (width 0.2) (layer "F.Cu") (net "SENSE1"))
 (segment (start 186.7163 138.2837) (end 186.7163 134.1228) (width 0.2) (layer "B.Cu") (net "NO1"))
 (segment (start 160 106.5903) (end 160 103.84) (width 0.2) (layer "B.Cu") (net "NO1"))
 (segment (start 171.0672 118.4737) (end 171.0672 117.3475) (width 0.2) (layer "B.Cu") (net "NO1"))
 (segment (start 168.8297 115.42) (end 160 106.5903) (width 0.2) (layer "B.Cu") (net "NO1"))
 (segment (start 171.0672 117.3475) (end 169.1397 115.42) (width 0.2) (layer "B.Cu") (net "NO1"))
 (segment (start 185 140) (end 186.7163 138.2837) (width 0.2) (layer "B.Cu") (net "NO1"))
 (segment (start 186.7163 134.1228) (end 171.0672 118.4737) (width 0.2) (layer "B.Cu") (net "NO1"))
 (segment (start 169.1397 115.42) (end 168.8297 115.42) (width 0.2) (layer "B.Cu") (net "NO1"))
 (segment (start 150 153) (end 160 153) (width 0.2) (layer "F.Cu") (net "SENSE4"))
 (segment (start 139.759 140.67) (end 150 150.911) (width 0.2) (layer "B.Cu") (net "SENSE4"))
 (segment (start 127.97 140.67) (end 139.759 140.67) (width 0.2) (layer "B.Cu") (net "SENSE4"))
 (segment (start 150 150.911) (end 150 153) (width 0.2) (layer "B.Cu") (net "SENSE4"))
 (segment (start 114 126.7) (end 127.97 140.67) (width 0.2) (layer "B.Cu") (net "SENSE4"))
 (segment (start 161.42 141.42) (end 175.9889 141.42) (width 0.2) (layer "F.Cu") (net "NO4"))
 (segment (start 160 142.84) (end 161.42 141.42) (width 0.2) (layer "F.Cu") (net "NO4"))
 (segment (start 186.7017 126.7017) (end 185 125) (width 0.2) (layer "F.Cu") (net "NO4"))
 (segment (start 186.7017 130.7072) (end 186.7017 126.7017) (width 0.2) (layer "F.Cu") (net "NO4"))
 (segment (start 175.9889 141.42) (end 186.7017 130.7072) (width 0.2) (layer "F.Cu") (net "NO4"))
 (segment (start 183.16 116.84) (end 169 116.84) (width 0.2) (layer "F.Cu") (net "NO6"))
 (segment (start 185 115) (end 183.16 116.84) (width 0.2) (layer "F.Cu") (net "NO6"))
 (segment (start 111.9694 138.8906) (end 111.9694 154.2615) (width 0.2) (layer "B.Cu") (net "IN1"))
 (segment (start 111.9694 154.2615) (end 113.6179 155.91) (width 0.2) (layer "B.Cu") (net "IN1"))
 (segment (start 113.6179 155.91) (end 115.45 155.91) (width 0.2) (layer "B.Cu") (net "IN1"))
 (segment (start 115.45 155.91) (end 128.54 169) (width 0.2) (layer "B.Cu") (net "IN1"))
 (segment (start 114 136.86) (end 111.9694 138.8906) (width 0.2) (layer "B.Cu") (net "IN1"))
 (segment (start 115.45 153.37) (end 131.08 169) (width 0.2) (layer "B.Cu") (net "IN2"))
 (segment (start 113.6379 153.37) (end 115.45 153.37) (width 0.2) (layer "B.Cu") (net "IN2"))
 (segment (start 114 139.4) (end 112.391 141.009) (width 0.2) (layer "B.Cu") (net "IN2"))
 (segment (start 112.391 152.1231) (end 113.6379 153.37) (width 0.2) (layer "B.Cu") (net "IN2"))
 (segment (start 112.391 141.009) (end 112.391 152.1231) (width 0.2) (layer "B.Cu") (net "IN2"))
 (segment (start 112.8212 150.0133) (end 112.8212 143.1188) (width 0.2) (layer "B.Cu") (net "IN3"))
 (segment (start 133.62 169) (end 115.45 150.83) (width 0.2) (layer "B.Cu") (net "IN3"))
 (segment (start 112.8212 143.1188) (end 114 141.94) (width 0.2) (layer "B.Cu") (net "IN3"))
 (segment (start 115.45 150.83) (end 113.6379 150.83) (width 0.2) (layer "B.Cu") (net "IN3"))
 (segment (start 113.6379 150.83) (end 112.8212 150.0133) (width 0.2) (layer "B.Cu") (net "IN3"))
 (segment (start 136.16 169) (end 116.72 149.56) (width 0.2) (layer "B.Cu") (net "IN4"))
 (segment (start 116.72 149.56) (end 114 149.56) (width 0.2) (layer "B.Cu") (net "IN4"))
 (segment (start 115.3898 135.7098) (end 114 134.32) (width 0.2) (layer "B.Cu") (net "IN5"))
 (segment (start 115.3898 145.6898) (end 115.3898 135.7098) (width 0.2) (layer "B.Cu") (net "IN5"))
 (segment (start 138.7 169) (end 115.3898 145.6898) (width 0.2) (layer "B.Cu") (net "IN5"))
 (segment (start 141.24 169) (end 118.1389 145.8989) (width 0.2) (layer "B.Cu") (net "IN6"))
 (segment (start 118.1389 135.9189) (end 114 131.78) (width 0.2) (layer "B.Cu") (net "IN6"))
 (segment (start 118.1389 145.8989) (end 118.1389 135.9189) (width 0.2) (layer "B.Cu") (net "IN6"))
 (segment (start 118.5819 133.8219) (end 114 129.24) (width 0.2) (layer "B.Cu") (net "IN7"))
 (segment (start 118.5819 143.8019) (end 118.5819 133.8219) (width 0.2) (layer "B.Cu") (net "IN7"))
 (segment (start 143.78 169) (end 118.5819 143.8019) (width 0.2) (layer "B.Cu") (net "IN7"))
 (segment (start 143.081 163.221) (end 117.501 163.221) (width 0.2) (layer "F.Cu") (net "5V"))
 (segment (start 117.501 163.221) (end 114 159.72) (width 0.2) (layer "F.Cu") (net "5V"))
 (segment (start 148.86 169) (end 143.081 163.221) (width 0.2) (layer "F.Cu") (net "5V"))
 (segment (start 185.2991 142.84) (end 187.1384 141.0007) (width 0.2) (layer "B.Cu") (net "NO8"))
 (segment (start 187.1384 107.1384) (end 185 105) (width 0.2) (layer "B.Cu") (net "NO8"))
 (segment (start 169 142.84) (end 185.2991 142.84) (width 0.2) (layer "B.Cu") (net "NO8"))
 (segment (start 187.1384 141.0007) (end 187.1384 107.1384) (width 0.2) (layer "B.Cu") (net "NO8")))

